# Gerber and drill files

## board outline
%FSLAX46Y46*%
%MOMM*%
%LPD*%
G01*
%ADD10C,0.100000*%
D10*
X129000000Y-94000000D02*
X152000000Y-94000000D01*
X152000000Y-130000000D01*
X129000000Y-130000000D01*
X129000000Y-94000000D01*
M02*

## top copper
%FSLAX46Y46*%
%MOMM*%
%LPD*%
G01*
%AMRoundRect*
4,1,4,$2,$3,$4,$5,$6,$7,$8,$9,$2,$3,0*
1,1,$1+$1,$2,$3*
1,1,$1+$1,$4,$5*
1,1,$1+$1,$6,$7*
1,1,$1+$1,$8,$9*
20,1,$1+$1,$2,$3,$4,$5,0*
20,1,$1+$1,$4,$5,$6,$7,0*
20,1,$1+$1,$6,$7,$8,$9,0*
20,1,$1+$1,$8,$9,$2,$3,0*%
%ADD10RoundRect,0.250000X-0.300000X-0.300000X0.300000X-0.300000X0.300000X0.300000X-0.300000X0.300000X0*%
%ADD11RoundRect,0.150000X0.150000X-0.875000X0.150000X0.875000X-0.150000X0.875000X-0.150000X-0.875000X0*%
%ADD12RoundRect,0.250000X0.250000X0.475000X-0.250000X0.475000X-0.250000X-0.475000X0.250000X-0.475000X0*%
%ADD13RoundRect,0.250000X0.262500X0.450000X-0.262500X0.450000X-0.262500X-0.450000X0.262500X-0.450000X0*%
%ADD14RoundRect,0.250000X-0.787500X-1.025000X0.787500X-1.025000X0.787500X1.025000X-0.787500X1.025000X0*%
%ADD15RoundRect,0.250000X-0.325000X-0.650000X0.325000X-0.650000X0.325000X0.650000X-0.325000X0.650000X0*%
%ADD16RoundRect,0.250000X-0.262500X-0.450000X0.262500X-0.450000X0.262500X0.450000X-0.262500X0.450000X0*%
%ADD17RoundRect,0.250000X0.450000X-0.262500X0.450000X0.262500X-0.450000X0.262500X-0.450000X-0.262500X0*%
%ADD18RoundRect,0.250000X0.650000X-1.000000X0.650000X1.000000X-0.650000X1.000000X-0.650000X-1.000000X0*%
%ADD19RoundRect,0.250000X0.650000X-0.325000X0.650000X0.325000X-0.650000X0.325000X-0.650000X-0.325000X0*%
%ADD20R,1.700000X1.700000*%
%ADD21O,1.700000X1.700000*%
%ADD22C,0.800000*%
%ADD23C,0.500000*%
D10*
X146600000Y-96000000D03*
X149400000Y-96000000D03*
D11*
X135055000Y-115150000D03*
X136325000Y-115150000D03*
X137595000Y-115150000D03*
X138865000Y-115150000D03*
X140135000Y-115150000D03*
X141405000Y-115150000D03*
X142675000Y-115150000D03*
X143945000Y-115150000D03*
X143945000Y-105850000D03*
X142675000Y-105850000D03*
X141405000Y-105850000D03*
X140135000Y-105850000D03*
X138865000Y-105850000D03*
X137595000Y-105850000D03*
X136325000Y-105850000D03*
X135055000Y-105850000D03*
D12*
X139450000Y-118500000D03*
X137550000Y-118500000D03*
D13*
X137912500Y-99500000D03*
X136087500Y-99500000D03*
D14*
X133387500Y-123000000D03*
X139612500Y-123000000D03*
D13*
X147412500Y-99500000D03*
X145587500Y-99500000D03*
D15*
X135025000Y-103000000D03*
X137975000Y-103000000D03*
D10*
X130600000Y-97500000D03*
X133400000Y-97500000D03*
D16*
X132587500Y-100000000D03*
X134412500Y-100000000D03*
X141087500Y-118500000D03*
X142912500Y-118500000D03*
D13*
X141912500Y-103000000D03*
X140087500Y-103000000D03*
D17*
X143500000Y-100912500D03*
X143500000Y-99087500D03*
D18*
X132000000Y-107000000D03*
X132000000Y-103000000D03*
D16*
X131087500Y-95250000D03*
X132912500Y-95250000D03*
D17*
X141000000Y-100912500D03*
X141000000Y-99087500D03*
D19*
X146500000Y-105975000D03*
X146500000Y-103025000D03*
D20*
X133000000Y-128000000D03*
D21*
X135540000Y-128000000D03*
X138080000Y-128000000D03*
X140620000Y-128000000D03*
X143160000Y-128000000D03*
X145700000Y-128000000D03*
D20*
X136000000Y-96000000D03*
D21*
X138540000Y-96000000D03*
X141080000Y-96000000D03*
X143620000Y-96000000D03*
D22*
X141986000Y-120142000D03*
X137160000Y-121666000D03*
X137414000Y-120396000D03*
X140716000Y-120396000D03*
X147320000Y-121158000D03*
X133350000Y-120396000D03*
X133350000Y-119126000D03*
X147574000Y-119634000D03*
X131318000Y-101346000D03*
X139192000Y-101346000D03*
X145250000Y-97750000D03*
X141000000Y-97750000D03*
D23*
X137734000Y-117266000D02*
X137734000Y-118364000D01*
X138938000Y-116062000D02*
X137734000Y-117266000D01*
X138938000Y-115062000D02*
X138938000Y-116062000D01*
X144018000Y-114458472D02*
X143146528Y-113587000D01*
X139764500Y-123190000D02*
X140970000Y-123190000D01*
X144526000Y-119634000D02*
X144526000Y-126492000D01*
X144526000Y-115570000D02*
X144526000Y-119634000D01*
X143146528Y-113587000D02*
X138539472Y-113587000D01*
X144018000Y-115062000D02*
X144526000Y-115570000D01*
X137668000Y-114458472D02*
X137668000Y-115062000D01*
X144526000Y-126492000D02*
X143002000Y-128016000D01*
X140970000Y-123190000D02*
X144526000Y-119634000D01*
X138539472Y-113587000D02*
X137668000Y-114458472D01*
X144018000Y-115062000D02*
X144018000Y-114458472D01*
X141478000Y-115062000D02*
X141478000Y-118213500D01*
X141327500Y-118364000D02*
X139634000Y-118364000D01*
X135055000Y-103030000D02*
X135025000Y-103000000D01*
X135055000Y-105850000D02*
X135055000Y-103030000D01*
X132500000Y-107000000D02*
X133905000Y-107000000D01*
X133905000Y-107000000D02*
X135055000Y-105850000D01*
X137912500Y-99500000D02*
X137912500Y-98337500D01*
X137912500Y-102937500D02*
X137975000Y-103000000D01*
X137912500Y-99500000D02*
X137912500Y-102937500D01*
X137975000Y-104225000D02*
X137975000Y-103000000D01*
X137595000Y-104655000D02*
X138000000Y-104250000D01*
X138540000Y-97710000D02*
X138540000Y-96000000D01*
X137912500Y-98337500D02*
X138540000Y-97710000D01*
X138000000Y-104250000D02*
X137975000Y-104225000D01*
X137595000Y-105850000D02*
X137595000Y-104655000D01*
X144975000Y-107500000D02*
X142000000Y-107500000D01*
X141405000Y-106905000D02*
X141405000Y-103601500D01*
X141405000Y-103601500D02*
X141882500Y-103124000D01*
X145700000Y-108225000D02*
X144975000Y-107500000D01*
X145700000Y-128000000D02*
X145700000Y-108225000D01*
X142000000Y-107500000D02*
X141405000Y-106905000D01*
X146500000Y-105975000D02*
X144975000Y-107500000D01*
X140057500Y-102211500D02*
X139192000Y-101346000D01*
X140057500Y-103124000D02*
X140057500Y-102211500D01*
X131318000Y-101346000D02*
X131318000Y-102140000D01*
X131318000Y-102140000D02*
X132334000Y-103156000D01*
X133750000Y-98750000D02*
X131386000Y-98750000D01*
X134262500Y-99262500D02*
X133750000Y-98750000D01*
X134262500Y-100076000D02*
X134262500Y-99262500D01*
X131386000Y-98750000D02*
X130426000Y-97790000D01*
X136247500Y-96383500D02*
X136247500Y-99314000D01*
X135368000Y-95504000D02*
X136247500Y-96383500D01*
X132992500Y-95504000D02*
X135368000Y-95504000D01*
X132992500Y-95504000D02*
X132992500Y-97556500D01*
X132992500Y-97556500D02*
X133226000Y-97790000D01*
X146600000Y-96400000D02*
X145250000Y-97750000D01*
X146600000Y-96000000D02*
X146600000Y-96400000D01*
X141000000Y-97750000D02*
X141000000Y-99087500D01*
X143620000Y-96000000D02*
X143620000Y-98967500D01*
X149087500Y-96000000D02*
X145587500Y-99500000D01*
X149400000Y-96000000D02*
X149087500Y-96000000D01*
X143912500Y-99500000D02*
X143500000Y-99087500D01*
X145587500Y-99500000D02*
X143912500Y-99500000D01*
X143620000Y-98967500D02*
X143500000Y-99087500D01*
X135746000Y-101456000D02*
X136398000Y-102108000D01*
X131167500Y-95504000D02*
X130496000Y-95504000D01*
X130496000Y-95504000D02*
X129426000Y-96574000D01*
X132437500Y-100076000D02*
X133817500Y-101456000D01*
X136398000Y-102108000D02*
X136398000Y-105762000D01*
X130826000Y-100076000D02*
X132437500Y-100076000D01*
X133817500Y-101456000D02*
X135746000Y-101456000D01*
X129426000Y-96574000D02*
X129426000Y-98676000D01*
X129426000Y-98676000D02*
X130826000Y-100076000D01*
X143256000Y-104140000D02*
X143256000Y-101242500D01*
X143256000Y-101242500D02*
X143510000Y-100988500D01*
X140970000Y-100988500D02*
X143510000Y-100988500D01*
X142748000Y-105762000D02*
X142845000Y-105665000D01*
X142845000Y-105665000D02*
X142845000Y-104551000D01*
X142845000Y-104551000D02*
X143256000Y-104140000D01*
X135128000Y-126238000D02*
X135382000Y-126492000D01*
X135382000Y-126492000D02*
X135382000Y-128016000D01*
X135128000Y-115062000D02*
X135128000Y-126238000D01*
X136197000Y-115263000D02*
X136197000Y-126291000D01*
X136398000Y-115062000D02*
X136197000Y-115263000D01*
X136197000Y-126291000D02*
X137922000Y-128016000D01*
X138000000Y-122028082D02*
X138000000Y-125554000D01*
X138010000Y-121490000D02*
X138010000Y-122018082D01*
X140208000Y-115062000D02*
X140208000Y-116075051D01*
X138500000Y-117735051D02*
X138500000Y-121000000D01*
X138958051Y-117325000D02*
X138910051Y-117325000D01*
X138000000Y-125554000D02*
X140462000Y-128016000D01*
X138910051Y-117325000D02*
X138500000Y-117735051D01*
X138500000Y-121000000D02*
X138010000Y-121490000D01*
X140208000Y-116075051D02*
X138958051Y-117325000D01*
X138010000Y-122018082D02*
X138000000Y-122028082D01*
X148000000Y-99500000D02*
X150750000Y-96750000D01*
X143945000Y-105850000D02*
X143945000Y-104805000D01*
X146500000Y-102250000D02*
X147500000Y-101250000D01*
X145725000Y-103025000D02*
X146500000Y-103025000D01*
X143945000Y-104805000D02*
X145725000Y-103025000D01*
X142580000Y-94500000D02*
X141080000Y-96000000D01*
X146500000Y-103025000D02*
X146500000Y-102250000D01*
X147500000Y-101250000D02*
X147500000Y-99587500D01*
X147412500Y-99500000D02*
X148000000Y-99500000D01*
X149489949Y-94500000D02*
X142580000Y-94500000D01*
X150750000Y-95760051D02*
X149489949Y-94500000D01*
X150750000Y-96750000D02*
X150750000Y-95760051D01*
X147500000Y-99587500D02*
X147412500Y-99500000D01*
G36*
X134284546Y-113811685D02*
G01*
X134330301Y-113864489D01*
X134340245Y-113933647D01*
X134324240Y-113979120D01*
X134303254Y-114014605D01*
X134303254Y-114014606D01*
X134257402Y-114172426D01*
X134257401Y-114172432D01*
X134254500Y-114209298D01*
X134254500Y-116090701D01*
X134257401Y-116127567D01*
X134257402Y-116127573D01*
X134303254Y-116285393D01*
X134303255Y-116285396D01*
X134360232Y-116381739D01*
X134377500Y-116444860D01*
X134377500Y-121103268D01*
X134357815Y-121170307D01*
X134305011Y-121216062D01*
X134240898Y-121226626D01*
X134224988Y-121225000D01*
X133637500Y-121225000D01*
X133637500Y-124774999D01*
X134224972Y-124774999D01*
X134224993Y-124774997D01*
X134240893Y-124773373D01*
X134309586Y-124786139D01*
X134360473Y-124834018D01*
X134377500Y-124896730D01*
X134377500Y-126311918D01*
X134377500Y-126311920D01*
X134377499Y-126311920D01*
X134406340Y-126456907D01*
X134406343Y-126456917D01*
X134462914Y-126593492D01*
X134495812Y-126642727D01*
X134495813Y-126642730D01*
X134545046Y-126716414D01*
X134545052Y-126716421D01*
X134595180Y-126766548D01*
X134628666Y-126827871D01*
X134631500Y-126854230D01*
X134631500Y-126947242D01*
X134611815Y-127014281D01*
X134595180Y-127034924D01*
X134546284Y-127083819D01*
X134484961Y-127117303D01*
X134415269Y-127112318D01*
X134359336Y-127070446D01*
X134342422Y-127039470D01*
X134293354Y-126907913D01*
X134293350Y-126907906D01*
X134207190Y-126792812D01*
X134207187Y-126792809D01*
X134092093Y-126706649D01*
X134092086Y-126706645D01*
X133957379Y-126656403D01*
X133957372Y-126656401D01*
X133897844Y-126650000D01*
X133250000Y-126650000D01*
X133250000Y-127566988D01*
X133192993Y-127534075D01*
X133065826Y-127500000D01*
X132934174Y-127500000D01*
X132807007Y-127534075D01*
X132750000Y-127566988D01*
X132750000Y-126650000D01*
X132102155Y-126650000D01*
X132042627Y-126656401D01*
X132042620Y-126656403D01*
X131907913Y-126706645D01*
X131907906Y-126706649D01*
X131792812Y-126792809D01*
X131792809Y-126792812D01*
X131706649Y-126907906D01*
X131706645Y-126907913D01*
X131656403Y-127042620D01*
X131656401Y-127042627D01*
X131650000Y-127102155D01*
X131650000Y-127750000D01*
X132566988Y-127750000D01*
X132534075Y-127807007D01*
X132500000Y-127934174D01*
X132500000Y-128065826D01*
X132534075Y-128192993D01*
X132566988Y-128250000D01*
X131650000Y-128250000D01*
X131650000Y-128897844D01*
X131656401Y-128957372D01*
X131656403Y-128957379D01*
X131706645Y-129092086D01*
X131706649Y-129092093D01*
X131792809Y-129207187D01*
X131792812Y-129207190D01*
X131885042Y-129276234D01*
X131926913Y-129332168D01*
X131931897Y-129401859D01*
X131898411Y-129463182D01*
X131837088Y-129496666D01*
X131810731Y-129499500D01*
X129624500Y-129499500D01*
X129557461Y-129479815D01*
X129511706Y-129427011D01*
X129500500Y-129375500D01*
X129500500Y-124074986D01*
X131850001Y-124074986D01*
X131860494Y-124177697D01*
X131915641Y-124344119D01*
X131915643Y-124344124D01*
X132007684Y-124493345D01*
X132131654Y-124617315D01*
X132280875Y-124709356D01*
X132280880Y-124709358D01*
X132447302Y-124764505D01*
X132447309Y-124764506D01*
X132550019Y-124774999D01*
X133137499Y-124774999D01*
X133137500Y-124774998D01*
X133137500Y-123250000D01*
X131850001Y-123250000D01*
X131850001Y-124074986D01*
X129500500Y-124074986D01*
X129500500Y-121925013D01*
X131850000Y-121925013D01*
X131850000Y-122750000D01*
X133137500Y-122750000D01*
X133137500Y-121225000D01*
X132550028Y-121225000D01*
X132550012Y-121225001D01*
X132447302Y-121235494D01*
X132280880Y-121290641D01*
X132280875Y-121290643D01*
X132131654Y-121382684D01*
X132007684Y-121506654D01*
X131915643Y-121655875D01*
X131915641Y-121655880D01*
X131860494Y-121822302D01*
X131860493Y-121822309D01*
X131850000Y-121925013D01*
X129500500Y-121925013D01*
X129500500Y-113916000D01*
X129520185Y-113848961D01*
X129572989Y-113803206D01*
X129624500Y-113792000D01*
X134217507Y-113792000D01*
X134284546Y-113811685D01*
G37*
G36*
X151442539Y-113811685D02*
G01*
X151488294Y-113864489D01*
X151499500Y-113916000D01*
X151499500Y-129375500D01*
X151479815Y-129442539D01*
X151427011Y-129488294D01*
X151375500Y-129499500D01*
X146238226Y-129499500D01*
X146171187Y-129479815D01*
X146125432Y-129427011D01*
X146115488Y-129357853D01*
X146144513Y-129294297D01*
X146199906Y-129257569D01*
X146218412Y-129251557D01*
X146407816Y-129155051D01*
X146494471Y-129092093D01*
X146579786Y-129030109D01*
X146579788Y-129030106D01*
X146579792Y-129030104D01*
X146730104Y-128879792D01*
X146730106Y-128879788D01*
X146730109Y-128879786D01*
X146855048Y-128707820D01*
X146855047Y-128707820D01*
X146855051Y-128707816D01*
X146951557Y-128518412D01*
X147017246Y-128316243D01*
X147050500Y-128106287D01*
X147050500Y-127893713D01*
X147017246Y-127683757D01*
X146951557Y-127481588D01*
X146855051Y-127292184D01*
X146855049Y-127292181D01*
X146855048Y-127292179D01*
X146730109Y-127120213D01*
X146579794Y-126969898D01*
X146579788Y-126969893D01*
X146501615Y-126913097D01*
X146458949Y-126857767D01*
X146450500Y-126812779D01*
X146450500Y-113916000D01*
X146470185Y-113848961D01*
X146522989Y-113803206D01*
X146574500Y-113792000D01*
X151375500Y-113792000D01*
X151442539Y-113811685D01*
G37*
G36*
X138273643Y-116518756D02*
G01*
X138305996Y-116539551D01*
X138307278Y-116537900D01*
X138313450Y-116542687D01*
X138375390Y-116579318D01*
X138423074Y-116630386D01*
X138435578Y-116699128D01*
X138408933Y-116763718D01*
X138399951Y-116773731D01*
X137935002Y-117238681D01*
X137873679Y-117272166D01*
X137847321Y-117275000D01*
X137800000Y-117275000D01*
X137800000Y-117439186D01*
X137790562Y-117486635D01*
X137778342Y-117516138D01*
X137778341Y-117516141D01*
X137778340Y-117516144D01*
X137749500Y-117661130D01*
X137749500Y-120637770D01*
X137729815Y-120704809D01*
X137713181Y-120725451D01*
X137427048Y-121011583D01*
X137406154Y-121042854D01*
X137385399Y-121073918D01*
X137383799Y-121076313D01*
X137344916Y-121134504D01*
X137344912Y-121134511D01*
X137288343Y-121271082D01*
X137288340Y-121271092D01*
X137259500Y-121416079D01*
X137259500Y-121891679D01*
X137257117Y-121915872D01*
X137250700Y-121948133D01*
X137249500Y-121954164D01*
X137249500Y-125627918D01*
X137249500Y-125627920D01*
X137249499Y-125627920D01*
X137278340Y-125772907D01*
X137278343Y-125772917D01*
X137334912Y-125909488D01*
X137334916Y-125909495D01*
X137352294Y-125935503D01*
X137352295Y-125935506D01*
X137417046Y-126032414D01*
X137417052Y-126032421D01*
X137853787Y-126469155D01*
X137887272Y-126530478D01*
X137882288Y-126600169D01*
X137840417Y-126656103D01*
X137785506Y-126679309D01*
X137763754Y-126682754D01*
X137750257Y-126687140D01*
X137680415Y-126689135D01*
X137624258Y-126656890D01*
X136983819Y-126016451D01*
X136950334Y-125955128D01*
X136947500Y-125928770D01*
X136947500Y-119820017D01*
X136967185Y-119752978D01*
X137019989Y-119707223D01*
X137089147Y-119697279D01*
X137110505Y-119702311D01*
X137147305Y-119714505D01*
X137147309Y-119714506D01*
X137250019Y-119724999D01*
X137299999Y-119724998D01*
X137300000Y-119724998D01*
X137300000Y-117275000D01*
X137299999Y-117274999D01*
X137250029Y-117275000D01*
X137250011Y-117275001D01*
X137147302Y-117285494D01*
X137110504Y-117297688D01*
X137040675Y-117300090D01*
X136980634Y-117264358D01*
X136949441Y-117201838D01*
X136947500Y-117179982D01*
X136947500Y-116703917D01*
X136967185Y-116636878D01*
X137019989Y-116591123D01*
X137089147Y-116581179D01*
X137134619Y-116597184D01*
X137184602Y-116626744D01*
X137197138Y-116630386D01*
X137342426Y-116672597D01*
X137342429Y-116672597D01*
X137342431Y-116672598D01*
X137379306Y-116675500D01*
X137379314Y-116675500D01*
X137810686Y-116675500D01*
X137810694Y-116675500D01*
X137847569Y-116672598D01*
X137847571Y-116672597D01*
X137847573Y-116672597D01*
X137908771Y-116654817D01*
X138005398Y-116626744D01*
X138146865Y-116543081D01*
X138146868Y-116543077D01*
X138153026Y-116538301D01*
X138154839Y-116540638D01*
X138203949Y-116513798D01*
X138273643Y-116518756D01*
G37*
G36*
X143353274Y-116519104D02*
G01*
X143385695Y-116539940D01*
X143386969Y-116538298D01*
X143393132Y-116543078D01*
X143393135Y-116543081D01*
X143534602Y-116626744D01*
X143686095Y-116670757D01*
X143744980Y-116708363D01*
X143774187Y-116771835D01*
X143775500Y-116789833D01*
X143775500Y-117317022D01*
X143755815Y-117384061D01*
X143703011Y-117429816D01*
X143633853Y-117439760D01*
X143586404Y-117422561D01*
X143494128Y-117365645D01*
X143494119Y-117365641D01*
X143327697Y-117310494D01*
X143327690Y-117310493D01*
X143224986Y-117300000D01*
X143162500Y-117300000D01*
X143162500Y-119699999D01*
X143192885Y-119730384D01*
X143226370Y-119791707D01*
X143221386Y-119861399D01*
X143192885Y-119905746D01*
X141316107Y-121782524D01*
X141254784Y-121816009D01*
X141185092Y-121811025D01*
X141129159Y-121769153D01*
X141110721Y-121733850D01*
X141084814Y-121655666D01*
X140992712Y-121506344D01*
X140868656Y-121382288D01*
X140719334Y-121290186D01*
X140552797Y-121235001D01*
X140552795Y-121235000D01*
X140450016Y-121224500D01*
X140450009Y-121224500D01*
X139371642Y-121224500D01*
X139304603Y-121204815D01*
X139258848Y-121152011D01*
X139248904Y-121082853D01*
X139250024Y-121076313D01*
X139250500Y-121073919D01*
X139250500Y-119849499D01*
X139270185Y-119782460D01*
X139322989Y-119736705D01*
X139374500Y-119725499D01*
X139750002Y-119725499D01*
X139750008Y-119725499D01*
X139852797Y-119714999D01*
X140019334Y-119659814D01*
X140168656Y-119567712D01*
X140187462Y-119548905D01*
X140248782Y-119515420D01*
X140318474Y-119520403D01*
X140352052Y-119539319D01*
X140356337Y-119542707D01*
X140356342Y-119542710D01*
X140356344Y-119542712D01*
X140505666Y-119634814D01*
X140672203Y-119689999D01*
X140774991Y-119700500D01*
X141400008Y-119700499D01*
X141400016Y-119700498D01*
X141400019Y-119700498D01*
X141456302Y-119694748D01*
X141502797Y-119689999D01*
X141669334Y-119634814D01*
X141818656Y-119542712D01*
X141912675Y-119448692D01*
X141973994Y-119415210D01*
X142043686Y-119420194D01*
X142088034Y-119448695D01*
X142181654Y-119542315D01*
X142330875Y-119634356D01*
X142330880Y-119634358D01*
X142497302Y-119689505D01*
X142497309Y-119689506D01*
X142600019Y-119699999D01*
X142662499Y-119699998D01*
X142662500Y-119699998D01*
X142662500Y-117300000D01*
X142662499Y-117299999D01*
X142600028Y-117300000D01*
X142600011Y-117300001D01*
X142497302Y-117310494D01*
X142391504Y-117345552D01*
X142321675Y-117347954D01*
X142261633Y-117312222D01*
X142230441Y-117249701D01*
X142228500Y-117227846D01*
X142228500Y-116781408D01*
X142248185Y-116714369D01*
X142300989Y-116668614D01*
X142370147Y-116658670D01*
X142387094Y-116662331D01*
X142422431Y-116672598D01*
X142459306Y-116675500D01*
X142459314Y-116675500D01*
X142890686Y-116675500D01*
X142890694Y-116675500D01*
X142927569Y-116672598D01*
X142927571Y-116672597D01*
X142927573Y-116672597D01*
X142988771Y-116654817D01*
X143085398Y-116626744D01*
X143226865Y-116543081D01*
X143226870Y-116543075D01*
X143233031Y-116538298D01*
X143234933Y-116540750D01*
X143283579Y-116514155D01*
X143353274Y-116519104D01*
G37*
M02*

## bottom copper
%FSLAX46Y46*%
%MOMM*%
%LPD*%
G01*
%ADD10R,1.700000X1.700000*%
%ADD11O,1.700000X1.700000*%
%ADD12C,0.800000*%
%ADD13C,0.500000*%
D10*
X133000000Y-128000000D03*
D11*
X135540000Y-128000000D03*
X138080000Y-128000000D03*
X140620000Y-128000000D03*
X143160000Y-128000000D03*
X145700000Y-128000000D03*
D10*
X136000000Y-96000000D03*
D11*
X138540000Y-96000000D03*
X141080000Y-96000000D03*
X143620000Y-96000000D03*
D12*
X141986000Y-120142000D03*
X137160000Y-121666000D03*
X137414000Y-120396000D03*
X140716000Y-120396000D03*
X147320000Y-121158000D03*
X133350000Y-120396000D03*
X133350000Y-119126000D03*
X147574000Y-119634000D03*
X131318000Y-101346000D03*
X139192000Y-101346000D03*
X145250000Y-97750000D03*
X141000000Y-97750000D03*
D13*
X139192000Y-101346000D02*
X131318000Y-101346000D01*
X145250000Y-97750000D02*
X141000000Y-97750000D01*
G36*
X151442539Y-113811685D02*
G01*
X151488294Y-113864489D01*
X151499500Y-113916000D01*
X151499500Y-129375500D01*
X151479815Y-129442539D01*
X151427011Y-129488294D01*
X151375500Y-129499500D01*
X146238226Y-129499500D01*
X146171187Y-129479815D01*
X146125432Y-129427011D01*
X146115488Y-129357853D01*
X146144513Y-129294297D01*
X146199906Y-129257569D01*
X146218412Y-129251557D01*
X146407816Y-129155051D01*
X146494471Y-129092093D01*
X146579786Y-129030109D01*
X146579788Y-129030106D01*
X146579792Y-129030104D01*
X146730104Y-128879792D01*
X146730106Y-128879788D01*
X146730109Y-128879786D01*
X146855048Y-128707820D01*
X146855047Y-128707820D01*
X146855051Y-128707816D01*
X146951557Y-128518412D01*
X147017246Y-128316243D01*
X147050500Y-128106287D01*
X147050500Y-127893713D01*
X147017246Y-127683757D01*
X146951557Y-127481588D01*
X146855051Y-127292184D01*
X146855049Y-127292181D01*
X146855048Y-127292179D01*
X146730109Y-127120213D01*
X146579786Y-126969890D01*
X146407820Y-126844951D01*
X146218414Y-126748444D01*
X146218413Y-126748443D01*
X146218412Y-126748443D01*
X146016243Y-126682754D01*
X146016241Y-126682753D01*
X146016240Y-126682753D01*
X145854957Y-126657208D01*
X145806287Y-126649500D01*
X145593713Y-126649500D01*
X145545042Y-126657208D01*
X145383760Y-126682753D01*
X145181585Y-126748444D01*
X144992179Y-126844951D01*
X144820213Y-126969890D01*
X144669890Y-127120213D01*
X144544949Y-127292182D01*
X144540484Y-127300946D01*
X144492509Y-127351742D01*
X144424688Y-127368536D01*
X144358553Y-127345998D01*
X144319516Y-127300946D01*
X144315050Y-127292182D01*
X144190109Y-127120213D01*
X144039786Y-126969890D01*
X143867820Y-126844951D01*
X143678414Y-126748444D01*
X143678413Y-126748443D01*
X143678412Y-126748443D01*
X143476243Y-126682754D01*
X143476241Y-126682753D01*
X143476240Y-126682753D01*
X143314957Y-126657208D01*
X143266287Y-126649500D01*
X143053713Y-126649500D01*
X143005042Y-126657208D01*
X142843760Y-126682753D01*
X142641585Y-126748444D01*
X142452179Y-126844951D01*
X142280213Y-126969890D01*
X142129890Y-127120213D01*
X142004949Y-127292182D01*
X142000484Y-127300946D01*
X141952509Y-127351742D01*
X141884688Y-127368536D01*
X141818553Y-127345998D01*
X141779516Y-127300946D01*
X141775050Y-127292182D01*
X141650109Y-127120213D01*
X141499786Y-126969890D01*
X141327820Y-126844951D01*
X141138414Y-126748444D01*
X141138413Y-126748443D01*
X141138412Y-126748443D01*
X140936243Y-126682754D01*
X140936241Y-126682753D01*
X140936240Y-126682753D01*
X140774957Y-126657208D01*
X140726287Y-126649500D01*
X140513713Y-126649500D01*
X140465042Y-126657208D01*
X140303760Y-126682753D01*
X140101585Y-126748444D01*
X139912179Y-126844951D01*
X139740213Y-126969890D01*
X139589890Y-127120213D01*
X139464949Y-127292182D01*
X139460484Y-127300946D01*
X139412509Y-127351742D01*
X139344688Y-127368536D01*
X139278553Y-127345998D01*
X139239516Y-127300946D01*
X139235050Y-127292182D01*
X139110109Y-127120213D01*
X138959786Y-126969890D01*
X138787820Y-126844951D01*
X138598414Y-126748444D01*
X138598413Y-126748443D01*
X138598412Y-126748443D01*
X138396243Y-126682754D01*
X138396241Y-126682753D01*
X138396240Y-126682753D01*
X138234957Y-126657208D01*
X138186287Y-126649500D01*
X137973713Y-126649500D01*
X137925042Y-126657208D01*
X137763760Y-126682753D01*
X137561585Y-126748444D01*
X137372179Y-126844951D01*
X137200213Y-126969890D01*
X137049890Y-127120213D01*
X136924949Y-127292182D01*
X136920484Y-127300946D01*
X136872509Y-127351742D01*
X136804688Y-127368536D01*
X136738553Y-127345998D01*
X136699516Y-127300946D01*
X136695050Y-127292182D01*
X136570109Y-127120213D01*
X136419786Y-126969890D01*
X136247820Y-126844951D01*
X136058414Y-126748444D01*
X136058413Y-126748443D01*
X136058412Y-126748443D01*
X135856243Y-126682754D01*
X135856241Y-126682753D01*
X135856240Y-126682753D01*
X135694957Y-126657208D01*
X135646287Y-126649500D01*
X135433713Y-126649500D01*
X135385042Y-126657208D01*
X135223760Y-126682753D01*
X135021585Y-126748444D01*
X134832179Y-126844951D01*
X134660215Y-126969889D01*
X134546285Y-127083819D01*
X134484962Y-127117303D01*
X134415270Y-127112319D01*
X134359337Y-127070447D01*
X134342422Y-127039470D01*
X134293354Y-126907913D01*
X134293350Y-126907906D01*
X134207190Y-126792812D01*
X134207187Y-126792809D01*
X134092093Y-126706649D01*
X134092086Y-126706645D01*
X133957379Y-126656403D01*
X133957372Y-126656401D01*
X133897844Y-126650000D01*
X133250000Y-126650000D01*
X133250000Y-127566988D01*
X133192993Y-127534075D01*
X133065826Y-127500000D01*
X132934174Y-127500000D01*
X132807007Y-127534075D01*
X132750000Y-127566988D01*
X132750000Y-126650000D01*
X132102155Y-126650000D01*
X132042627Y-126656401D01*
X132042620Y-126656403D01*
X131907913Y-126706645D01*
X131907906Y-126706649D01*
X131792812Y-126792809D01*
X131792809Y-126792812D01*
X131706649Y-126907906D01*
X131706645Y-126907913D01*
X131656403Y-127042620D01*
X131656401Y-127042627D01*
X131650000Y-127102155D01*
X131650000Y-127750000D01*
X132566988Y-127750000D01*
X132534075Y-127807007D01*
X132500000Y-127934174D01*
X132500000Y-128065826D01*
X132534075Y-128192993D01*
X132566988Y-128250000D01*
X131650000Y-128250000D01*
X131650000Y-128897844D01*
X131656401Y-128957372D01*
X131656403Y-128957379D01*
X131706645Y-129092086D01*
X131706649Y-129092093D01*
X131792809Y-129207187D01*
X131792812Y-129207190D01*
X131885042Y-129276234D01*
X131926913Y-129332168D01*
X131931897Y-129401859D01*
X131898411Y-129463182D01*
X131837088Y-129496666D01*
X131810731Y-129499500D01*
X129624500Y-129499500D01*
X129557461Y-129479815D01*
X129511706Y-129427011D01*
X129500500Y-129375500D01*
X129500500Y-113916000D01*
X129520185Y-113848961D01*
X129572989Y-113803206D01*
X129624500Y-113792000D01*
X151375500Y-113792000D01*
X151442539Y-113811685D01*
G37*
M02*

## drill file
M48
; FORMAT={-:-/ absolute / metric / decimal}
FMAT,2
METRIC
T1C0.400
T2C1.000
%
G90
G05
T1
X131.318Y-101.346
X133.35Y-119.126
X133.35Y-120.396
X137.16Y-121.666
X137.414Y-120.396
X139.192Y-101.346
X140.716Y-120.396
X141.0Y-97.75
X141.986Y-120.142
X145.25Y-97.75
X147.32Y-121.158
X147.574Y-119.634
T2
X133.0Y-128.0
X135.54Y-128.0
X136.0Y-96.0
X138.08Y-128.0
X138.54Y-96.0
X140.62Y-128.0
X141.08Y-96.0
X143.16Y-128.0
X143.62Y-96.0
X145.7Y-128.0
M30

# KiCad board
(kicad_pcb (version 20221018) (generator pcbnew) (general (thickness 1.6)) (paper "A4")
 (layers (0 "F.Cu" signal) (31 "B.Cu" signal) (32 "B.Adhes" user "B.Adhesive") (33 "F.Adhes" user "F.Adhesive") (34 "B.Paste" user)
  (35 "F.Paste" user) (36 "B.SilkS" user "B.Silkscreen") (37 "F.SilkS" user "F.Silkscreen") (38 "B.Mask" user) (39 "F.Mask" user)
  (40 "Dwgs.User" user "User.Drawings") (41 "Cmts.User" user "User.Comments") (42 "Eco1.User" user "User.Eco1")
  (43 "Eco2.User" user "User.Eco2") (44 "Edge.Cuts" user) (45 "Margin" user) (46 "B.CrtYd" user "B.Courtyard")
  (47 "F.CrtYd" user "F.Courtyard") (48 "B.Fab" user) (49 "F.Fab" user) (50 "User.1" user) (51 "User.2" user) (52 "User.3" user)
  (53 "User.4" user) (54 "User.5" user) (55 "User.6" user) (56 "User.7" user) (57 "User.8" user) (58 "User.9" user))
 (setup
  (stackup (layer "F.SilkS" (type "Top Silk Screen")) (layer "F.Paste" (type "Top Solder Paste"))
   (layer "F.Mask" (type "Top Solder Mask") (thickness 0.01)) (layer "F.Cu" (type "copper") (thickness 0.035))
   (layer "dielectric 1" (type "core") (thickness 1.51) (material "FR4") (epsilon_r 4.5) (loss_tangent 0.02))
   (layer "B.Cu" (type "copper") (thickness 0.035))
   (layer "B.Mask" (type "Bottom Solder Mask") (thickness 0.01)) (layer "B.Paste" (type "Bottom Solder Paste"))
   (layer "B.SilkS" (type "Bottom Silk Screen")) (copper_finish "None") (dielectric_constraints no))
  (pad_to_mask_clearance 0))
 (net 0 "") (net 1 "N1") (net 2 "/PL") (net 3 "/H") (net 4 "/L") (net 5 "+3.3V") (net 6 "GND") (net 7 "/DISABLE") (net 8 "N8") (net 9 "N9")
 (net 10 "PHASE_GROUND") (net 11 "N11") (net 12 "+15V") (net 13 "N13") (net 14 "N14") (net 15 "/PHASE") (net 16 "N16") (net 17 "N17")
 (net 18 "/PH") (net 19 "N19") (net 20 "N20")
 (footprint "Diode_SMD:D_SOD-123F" (layer "F.Cu") (at 148 96)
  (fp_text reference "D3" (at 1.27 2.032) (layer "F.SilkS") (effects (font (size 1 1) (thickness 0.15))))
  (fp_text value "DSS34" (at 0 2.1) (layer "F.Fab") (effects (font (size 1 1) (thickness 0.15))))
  (pad "1" smd roundrect (at -1.4 0) (size 1.1 1.1) (layers "F.Cu" "F.Paste" "F.Mask") (roundrect_rratio 0.2272727273) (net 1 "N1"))
  (pad "2" smd roundrect (at 1.4 0) (size 1.1 1.1) (layers "F.Cu" "F.Paste" "F.Mask") (roundrect_rratio 0.2272727273) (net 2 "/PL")))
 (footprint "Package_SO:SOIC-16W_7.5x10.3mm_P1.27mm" (layer "F.Cu") (at 139.5 110.5 90)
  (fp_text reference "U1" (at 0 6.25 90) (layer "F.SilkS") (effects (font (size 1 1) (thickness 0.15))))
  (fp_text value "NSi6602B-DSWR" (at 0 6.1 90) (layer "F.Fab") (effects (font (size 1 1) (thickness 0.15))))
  (pad "1" smd roundrect (at -4.65 -4.445 90) (size 2.05 0.6) (layers "F.Cu" "F.Paste" "F.Mask") (roundrect_rratio 0.25) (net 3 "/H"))
  (pad "2" smd roundrect (at -4.65 -3.175 90) (size 2.05 0.6) (layers "F.Cu" "F.Paste" "F.Mask") (roundrect_rratio 0.25) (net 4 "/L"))
  (pad "3" smd roundrect (at -4.65 -1.905 90) (size 2.05 0.6) (layers "F.Cu" "F.Paste" "F.Mask") (roundrect_rratio 0.25) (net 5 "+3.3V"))
  (pad "4" smd roundrect (at -4.65 -0.635 90) (size 2.05 0.6) (layers "F.Cu" "F.Paste" "F.Mask") (roundrect_rratio 0.25) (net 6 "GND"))
  (pad "5" smd roundrect (at -4.65 0.635 90) (size 2.05 0.6) (layers "F.Cu" "F.Paste" "F.Mask") (roundrect_rratio 0.25) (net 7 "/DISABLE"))
  (pad "6" smd roundrect (at -4.65 1.905 90) (size 2.05 0.6) (layers "F.Cu" "F.Paste" "F.Mask") (roundrect_rratio 0.25) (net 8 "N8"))
  (pad "7" smd roundrect (at -4.65 3.175 90) (size 2.05 0.6) (layers "F.Cu" "F.Paste" "F.Mask") (roundrect_rratio 0.25) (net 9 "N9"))
  (pad "8" smd roundrect (at -4.65 4.445 90) (size 2.05 0.6) (layers "F.Cu" "F.Paste" "F.Mask") (roundrect_rratio 0.25) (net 5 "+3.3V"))
  (pad "9" smd roundrect (at 4.65 4.445 90) (size 2.05 0.6) (layers "F.Cu" "F.Paste" "F.Mask") (roundrect_rratio 0.25)
   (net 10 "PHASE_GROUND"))
  (pad "10" smd roundrect (at 4.65 3.175 90) (size 2.05 0.6) (layers "F.Cu" "F.Paste" "F.Mask") (roundrect_rratio 0.25) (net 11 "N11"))
  (pad "11" smd roundrect (at 4.65 1.905 90) (size 2.05 0.6) (layers "F.Cu" "F.Paste" "F.Mask") (roundrect_rratio 0.25) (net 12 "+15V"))
  (pad "12" smd roundrect (at 4.65 0.635 90) (size 2.05 0.6) (layers "F.Cu" "F.Paste" "F.Mask") (roundrect_rratio 0.25) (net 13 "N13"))
  (pad "13" smd roundrect (at 4.65 -0.635 90) (size 2.05 0.6) (layers "F.Cu" "F.Paste" "F.Mask") (roundrect_rratio 0.25) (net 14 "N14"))
  (pad "14" smd roundrect (at 4.65 -1.905 90) (size 2.05 0.6) (layers "F.Cu" "F.Paste" "F.Mask") (roundrect_rratio 0.25) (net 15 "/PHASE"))
  (pad "15" smd roundrect (at 4.65 -3.175 90) (size 2.05 0.6) (layers "F.Cu" "F.Paste" "F.Mask") (roundrect_rratio 0.25) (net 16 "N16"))
  (pad "16" smd roundrect (at 4.65 -4.445 90) (size 2.05 0.6) (layers "F.Cu" "F.Paste" "F.Mask") (roundrect_rratio 0.25) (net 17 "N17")))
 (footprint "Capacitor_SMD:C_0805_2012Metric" (layer "F.Cu") (at 138.5 118.5 180)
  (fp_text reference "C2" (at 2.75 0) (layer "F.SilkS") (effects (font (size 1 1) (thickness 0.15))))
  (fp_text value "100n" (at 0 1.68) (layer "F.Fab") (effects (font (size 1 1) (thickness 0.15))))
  (pad "1" smd roundrect (at -0.95 0 180) (size 1 1.45) (layers "F.Cu" "F.Paste" "F.Mask") (roundrect_rratio 0.25) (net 8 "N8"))
  (pad "2" smd roundrect (at 0.95 0 180) (size 1 1.45) (layers "F.Cu" "F.Paste" "F.Mask") (roundrect_rratio 0.25) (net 6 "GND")))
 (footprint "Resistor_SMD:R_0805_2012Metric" (layer "F.Cu") (at 137 99.5 180)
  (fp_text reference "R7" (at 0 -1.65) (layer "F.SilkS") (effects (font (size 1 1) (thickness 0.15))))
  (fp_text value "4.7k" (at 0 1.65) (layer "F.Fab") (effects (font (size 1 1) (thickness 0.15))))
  (pad "1" smd roundrect (at -0.9125 0 180) (size 1.025 1.4) (layers "F.Cu" "F.Paste" "F.Mask") (roundrect_rratio 0.243902)
   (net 15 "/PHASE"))
  (pad "2" smd roundrect (at 0.9125 0 180) (size 1.025 1.4) (layers "F.Cu" "F.Paste" "F.Mask") (roundrect_rratio 0.243902) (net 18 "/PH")))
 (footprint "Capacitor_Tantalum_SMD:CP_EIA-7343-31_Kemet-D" (layer "F.Cu") (at 136.5 123)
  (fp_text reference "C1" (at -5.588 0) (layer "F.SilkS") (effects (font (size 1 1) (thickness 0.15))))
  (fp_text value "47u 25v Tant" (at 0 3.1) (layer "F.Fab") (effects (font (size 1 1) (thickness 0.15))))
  (pad "1" smd roundrect (at -3.1125 0) (size 2.075 2.55) (layers "F.Cu" "F.Paste" "F.Mask") (roundrect_rratio 0.120482) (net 6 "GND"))
  (pad "2" smd roundrect (at 3.1125 0) (size 2.075 2.55) (layers "F.Cu" "F.Paste" "F.Mask") (roundrect_rratio 0.120482) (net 5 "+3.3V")))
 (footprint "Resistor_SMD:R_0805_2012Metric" (layer "F.Cu") (at 146.5 99.5 180)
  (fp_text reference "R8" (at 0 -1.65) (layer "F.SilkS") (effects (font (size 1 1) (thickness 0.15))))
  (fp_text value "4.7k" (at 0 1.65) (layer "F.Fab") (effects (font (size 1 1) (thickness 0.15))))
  (pad "1" smd roundrect (at -0.9125 0 180) (size 1.025 1.4) (layers "F.Cu" "F.Paste" "F.Mask") (roundrect_rratio 0.243902)
   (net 10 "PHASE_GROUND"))
  (pad "2" smd roundrect (at 0.9125 0 180) (size 1.025 1.4) (layers "F.Cu" "F.Paste" "F.Mask") (roundrect_rratio 0.243902) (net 2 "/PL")))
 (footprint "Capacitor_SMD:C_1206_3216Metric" (layer "F.Cu") (at 136.5 103)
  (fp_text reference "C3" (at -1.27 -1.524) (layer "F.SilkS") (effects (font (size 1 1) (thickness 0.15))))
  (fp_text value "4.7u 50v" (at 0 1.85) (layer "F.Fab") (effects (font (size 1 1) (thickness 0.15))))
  (pad "1" smd roundrect (at -1.475 0) (size 1.15 1.8) (layers "F.Cu" "F.Paste" "F.Mask") (roundrect_rratio 0.217391) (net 17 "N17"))
  (pad "2" smd roundrect (at 1.475 0) (size 1.15 1.8) (layers "F.Cu" "F.Paste" "F.Mask") (roundrect_rratio 0.217391) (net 15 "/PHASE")))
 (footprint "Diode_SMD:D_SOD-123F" (layer "F.Cu") (at 132 97.5)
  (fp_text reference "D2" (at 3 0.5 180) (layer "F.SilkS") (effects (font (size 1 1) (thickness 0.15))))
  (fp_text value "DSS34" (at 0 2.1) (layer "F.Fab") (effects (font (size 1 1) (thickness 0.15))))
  (pad "1" smd roundrect (at -1.4 0) (size 1.1 1.1) (layers "F.Cu" "F.Paste" "F.Mask") (roundrect_rratio 0.2272727273) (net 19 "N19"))
  (pad "2" smd roundrect (at 1.4 0) (size 1.1 1.1) (layers "F.Cu" "F.Paste" "F.Mask") (roundrect_rratio 0.2272727273) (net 18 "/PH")))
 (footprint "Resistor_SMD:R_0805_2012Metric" (layer "F.Cu") (at 133.5 100)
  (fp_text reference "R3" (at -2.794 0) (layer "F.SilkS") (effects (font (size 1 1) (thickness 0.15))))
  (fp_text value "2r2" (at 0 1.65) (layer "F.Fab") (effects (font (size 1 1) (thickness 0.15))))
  (pad "1" smd roundrect (at -0.9125 0) (size 1.025 1.4) (layers "F.Cu" "F.Paste" "F.Mask") (roundrect_rratio 0.243902) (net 16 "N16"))
  (pad "2" smd roundrect (at 0.9125 0) (size 1.025 1.4) (layers "F.Cu" "F.Paste" "F.Mask") (roundrect_rratio 0.243902) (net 19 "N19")))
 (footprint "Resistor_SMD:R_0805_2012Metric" (layer "F.Cu") (at 142 118.5)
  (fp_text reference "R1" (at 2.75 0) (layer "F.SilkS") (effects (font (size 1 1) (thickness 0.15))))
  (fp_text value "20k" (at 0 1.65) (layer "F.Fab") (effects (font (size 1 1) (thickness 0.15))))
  (pad "1" smd roundrect (at -0.9125 0) (size 1.025 1.4) (layers "F.Cu" "F.Paste" "F.Mask") (roundrect_rratio 0.243902) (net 8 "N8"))
  (pad "2" smd roundrect (at 0.9125 0) (size 1.025 1.4) (layers "F.Cu" "F.Paste" "F.Mask") (roundrect_rratio 0.243902) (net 6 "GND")))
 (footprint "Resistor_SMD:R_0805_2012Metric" (layer "F.Cu") (at 141 103 180)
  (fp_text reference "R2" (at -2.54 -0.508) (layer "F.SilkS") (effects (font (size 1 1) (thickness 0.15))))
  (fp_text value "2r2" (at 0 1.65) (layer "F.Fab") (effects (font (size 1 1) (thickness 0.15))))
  (pad "1" smd roundrect (at -0.9125 0 180) (size 1.025 1.4) (layers "F.Cu" "F.Paste" "F.Mask") (roundrect_rratio 0.243902) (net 12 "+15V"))
  (pad "2" smd roundrect (at 0.9125 0 180) (size 1.025 1.4) (layers "F.Cu" "F.Paste" "F.Mask") (roundrect_rratio 0.243902) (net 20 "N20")))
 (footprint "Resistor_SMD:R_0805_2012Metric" (layer "F.Cu") (at 143.5 100 90)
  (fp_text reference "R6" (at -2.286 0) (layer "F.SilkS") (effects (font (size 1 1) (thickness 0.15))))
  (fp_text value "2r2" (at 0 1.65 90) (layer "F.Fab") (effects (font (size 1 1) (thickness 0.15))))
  (pad "1" smd roundrect (at -0.9125 0 90) (size 1.025 1.4) (layers "F.Cu" "F.Paste" "F.Mask") (roundrect_rratio 0.243902) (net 11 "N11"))
  (pad "2" smd roundrect (at 0.9125 0 90) (size 1.025 1.4) (layers "F.Cu" "F.Paste" "F.Mask") (roundrect_rratio 0.243902) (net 2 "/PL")))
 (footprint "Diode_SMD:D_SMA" (layer "F.Cu") (at 132 105 90)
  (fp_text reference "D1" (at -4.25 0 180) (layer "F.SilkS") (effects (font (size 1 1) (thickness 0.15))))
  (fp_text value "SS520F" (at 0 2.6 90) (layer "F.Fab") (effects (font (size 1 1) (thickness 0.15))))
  (pad "1" smd roundrect (at -2 0 90) (size 2.5 1.8) (layers "F.Cu" "F.Paste" "F.Mask") (roundrect_rratio 0.1388888889) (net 17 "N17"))
  (pad "2" smd roundrect (at 2 0 90) (size 2.5 1.8) (layers "F.Cu" "F.Paste" "F.Mask") (roundrect_rratio 0.1388888889) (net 20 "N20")))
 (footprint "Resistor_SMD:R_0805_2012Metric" (layer "F.Cu") (at 132 95.25)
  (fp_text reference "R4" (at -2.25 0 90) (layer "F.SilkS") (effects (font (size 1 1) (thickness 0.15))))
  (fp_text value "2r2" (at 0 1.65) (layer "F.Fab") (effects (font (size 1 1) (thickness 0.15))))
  (pad "1" smd roundrect (at -0.9125 0) (size 1.025 1.4) (layers "F.Cu" "F.Paste" "F.Mask") (roundrect_rratio 0.243902) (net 16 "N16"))
  (pad "2" smd roundrect (at 0.9125 0) (size 1.025 1.4) (layers "F.Cu" "F.Paste" "F.Mask") (roundrect_rratio 0.243902) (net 18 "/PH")))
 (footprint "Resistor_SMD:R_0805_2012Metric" (layer "F.Cu") (at 141 100 90)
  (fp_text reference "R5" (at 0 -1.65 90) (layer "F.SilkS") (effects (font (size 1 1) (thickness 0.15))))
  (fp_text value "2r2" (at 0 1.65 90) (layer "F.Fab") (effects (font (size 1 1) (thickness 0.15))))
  (pad "1" smd roundrect (at -0.9125 0 90) (size 1.025 1.4) (layers "F.Cu" "F.Paste" "F.Mask") (roundrect_rratio 0.243902) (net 11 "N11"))
  (pad "2" smd roundrect (at 0.9125 0 90) (size 1.025 1.4) (layers "F.Cu" "F.Paste" "F.Mask") (roundrect_rratio 0.243902) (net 1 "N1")))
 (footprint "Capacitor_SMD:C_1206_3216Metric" (layer "F.Cu") (at 146.5 104.5 90)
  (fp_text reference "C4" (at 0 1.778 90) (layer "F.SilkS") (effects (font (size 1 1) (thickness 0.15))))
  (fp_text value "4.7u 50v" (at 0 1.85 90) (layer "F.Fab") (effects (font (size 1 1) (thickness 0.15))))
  (pad "1" smd roundrect (at -1.475 0 90) (size 1.15 1.8) (layers "F.Cu" "F.Paste" "F.Mask") (roundrect_rratio 0.217391) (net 12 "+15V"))
  (pad "2" smd roundrect (at 1.475 0 90) (size 1.15 1.8) (layers "F.Cu" "F.Paste" "F.Mask") (roundrect_rratio 0.217391)
   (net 10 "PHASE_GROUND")))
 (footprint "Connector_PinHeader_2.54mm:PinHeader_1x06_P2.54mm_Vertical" (layer "B.Cu") (at 133 128 -90)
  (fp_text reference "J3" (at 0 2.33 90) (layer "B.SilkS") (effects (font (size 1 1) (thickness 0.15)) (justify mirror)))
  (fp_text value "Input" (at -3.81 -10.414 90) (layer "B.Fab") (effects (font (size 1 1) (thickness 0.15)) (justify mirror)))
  (pad "1" thru_hole rect (at 0 0 270) (size 1.7 1.7) (drill 1) (layers "*.Cu" "*.Mask") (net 6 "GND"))
  (pad "2" thru_hole oval (at 0 -2.54 270) (size 1.7 1.7) (drill 1) (layers "*.Cu" "*.Mask") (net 3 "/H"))
  (pad "3" thru_hole oval (at 0 -5.08 270) (size 1.7 1.7) (drill 1) (layers "*.Cu" "*.Mask") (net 4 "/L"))
  (pad "4" thru_hole oval (at 0 -7.62 270) (size 1.7 1.7) (drill 1) (layers "*.Cu" "*.Mask") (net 7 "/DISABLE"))
  (pad "5" thru_hole oval (at 0 -10.16 270) (size 1.7 1.7) (drill 1) (layers "*.Cu" "*.Mask") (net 5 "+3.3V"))
  (pad "6" thru_hole oval (at 0 -12.7 270) (size 1.7 1.7) (drill 1) (layers "*.Cu" "*.Mask") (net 12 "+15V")))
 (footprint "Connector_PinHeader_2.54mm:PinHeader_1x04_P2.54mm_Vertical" (layer "B.Cu") (at 136 96 -90)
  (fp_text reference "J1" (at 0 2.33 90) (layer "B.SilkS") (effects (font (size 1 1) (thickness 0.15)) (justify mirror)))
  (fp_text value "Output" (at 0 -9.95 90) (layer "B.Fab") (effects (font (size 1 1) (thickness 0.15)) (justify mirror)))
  (pad "1" thru_hole rect (at 0 0 270) (size 1.7 1.7) (drill 1) (layers "*.Cu" "*.Mask") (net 18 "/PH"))
  (pad "2" thru_hole oval (at 0 -2.54 270) (size 1.7 1.7) (drill 1) (layers "*.Cu" "*.Mask") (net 15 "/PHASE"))
  (pad "3" thru_hole oval (at 0 -5.08 270) (size 1.7 1.7) (drill 1) (layers "*.Cu" "*.Mask") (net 10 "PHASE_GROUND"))
  (pad "4" thru_hole oval (at 0 -7.62 270) (size 1.7 1.7) (drill 1) (layers "*.Cu" "*.Mask") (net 2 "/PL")))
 (gr_rect (start 129 94) (end 152 130) (stroke (width 0.1) (type default)) (fill none) (layer "Edge.Cuts"))
 (segment (start 137.734 117.266) (end 137.734 118.364) (width 0.5) (layer "F.Cu") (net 6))
 (segment (start 138.938 116.062) (end 137.734 117.266) (width 0.5) (layer "F.Cu") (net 6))
 (segment (start 138.938 115.062) (end 138.938 116.062) (width 0.5) (layer "F.Cu") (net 6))
 (via (at 141.986 120.142) (size 0.8) (drill 0.4) (layers "F.Cu" "B.Cu") (free) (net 6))
 (via (at 137.16 121.666) (size 0.8) (drill 0.4) (layers "F.Cu" "B.Cu") (free) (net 6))
 (via (at 137.414 120.396) (size 0.8) (drill 0.4) (layers "F.Cu" "B.Cu") (free) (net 6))
 (via (at 140.716 120.396) (size 0.8) (drill 0.4) (layers "F.Cu" "B.Cu") (free) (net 6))
 (via (at 147.32 121.158) (size 0.8) (drill 0.4) (layers "F.Cu" "B.Cu") (free) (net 6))
 (via (at 133.35 120.396) (size 0.8) (drill 0.4) (layers "F.Cu" "B.Cu") (free) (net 6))
 (via (at 133.35 119.126) (size 0.8) (drill 0.4) (layers "F.Cu" "B.Cu") (free) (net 6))
 (via (at 147.574 119.634) (size 0.8) (drill 0.4) (layers "F.Cu" "B.Cu") (free) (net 6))
 (segment (start 144.018 114.458472) (end 143.146528 113.587) (width 0.5) (layer "F.Cu") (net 5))
 (segment (start 139.7645 123.19) (end 140.97 123.19) (width 0.5) (layer "F.Cu") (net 5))
 (segment (start 144.526 119.634) (end 144.526 126.492) (width 0.5) (layer "F.Cu") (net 5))
 (segment (start 144.526 115.57) (end 144.526 119.634) (width 0.5) (layer "F.Cu") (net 5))
 (segment (start 143.146528 113.587) (end 138.539472 113.587) (width 0.5) (layer "F.Cu") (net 5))
 (segment (start 144.018 115.062) (end 144.526 115.57) (width 0.5) (layer "F.Cu") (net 5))
 (segment (start 137.668 114.458472) (end 137.668 115.062) (width 0.5) (layer "F.Cu") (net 5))
 (segment (start 144.526 126.492) (end 143.002 128.016) (width 0.5) (layer "F.Cu") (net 5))
 (segment (start 140.97 123.19) (end 144.526 119.634) (width 0.5) (layer "F.Cu") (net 5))
 (segment (start 138.539472 113.587) (end 137.668 114.458472) (width 0.5) (layer "F.Cu") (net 5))
 (segment (start 144.018 115.062) (end 144.018 114.458472) (width 0.5) (layer "F.Cu") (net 5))
 (segment (start 141.478 115.062) (end 141.478 118.2135) (width 0.5) (layer "F.Cu") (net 8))
 (segment (start 141.3275 118.364) (end 139.634 118.364) (width 0.5) (layer "F.Cu") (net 8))
 (segment (start 135.055 103.03) (end 135.025 103) (width 0.5) (layer "F.Cu") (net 17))
 (segment (start 135.055 105.85) (end 135.055 103.03) (width 0.5) (layer "F.Cu") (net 17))
 (segment (start 132.5 107) (end 133.905 107) (width 0.5) (layer "F.Cu") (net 17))
 (segment (start 133.905 107) (end 135.055 105.85) (width 0.5) (layer "F.Cu") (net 17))
 (segment (start 137.9125 99.5) (end 137.9125 98.3375) (width 0.5) (layer "F.Cu") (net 15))
 (segment (start 137.9125 102.9375) (end 137.975 103) (width 0.5) (layer "F.Cu") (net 15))
 (segment (start 137.9125 99.5) (end 137.9125 102.9375) (width 0.5) (layer "F.Cu") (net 15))
 (segment (start 137.975 104.225) (end 137.975 103) (width 0.5) (layer "F.Cu") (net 15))
 (segment (start 137.595 104.655) (end 138 104.25) (width 0.5) (layer "F.Cu") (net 15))
 (segment (start 138.54 97.71) (end 138.54 96) (width 0.5) (layer "F.Cu") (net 15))
 (segment (start 137.9125 98.3375) (end 138.54 97.71) (width 0.5) (layer "F.Cu") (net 15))
 (segment (start 138 104.25) (end 137.975 104.225) (width 0.5) (layer "F.Cu") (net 15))
 (segment (start 137.595 105.85) (end 137.595 104.655) (width 0.5) (layer "F.Cu") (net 15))
 (segment (start 144.975 107.5) (end 142 107.5) (width 0.5) (layer "F.Cu") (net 12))
 (segment (start 141.405 106.905) (end 141.405 103.6015) (width 0.5) (layer "F.Cu") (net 12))
 (segment (start 141.405 103.6015) (end 141.8825 103.124) (width 0.5) (layer "F.Cu") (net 12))
 (segment (start 145.7 108.225) (end 144.975 107.5) (width 0.5) (layer "F.Cu") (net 12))
 (segment (start 145.7 128) (end 145.7 108.225) (width 0.5) (layer "F.Cu") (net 12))
 (segment (start 142 107.5) (end 141.405 106.905) (width 0.5) (layer "F.Cu") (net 12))
 (segment (start 146.5 105.975) (end 144.975 107.5) (width 0.5) (layer "F.Cu") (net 12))
 (segment (start 140.0575 102.2115) (end 139.192 101.346) (width 0.5) (layer "F.Cu") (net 20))
 (segment (start 140.0575 103.124) (end 140.0575 102.2115) (width 0.5) (layer "F.Cu") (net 20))
 (segment (start 131.318 101.346) (end 131.318 102.14) (width 0.5) (layer "F.Cu") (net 20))
 (segment (start 131.318 102.14) (end 132.334 103.156) (width 0.5) (layer "F.Cu") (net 20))
 (via (at 131.318 101.346) (size 0.8) (drill 0.4) (layers "F.Cu" "B.Cu") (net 20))
 (via (at 139.192 101.346) (size 0.8) (drill 0.4) (layers "F.Cu" "B.Cu") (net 20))
 (segment (start 139.192 101.346) (end 131.318 101.346) (width 0.5) (layer "B.Cu") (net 20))
 (segment (start 133.75 98.75) (end 131.386 98.75) (width 0.5) (layer "F.Cu") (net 19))
 (segment (start 134.2625 99.2625) (end 133.75 98.75) (width 0.5) (layer "F.Cu") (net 19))
 (segment (start 134.2625 100.076) (end 134.2625 99.2625) (width 0.5) (layer "F.Cu") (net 19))
 (segment (start 131.386 98.75) (end 130.426 97.79) (width 0.5) (layer "F.Cu") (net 19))
 (segment (start 136.2475 96.3835) (end 136.2475 99.314) (width 0.5) (layer "F.Cu") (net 18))
 (segment (start 135.368 95.504) (end 136.2475 96.3835) (width 0.5) (layer "F.Cu") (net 18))
 (segment (start 132.9925 95.504) (end 135.368 95.504) (width 0.5) (layer "F.Cu") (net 18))
 (segment (start 132.9925 95.504) (end 132.9925 97.5565) (width 0.5) (layer "F.Cu") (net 18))
 (segment (start 132.9925 97.5565) (end 133.226 97.79) (width 0.5) (layer "F.Cu") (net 18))
 (segment (start 146.6 96.4) (end 145.25 97.75) (width 0.5) (layer "F.Cu") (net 1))
 (segment (start 146.6 96) (end 146.6 96.4) (width 0.5) (layer "F.Cu") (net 1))
 (segment (start 141 97.75) (end 141 99.0875) (width 0.5) (layer "F.Cu") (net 1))
 (via (at 145.25 97.75) (size 0.8) (drill 0.4) (layers "F.Cu" "B.Cu") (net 1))
 (via (at 141 97.75) (size 0.8) (drill 0.4) (layers "F.Cu" "B.Cu") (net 1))
 (segment (start 145.25 97.75) (end 141 97.75) (width 0.5) (layer "B.Cu") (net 1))
 (segment (start 143.62 96) (end 143.62 98.9675) (width 0.5) (layer "F.Cu") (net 2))
 (segment (start 149.0875 96) (end 145.5875 99.5) (width 0.5) (layer "F.Cu") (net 2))
 (segment (start 149.4 96) (end 149.0875 96) (width 0.5) (layer "F.Cu") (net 2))
 (segment (start 143.9125 99.5) (end 143.5 99.0875) (width 0.5) (layer "F.Cu") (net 2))
 (segment (start 145.5875 99.5) (end 143.9125 99.5) (width 0.5) (layer "F.Cu") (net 2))
 (segment (start 143.62 98.9675) (end 143.5 99.0875) (width 0.5) (layer "F.Cu") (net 2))
 (segment (start 135.746 101.456) (end 136.398 102.108) (width 0.5) (layer "F.Cu") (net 16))
 (segment (start 131.1675 95.504) (end 130.496 95.504) (width 0.5) (layer "F.Cu") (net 16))
 (segment (start 130.496 95.504) (end 129.426 96.574) (width 0.5) (layer "F.Cu") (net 16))
 (segment (start 132.4375 100.076) (end 133.8175 101.456) (width 0.5) (layer "F.Cu") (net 16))
 (segment (start 136.398 102.108) (end 136.398 105.762) (width 0.5) (layer "F.Cu") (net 16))
 (segment (start 130.826 100.076) (end 132.4375 100.076) (width 0.5) (layer "F.Cu") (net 16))
 (segment (start 133.8175 101.456) (end 135.746 101.456) (width 0.5) (layer "F.Cu") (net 16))
 (segment (start 129.426 96.574) (end 129.426 98.676) (width 0.5) (layer "F.Cu") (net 16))
 (segment (start 129.426 98.676) (end 130.826 100.076) (width 0.5) (layer "F.Cu") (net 16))
 (segment (start 143.256 104.14) (end 143.256 101.2425) (width 0.5) (layer "F.Cu") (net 11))
 (segment (start 143.256 101.2425) (end 143.51 100.9885) (width 0.5) (layer "F.Cu") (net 11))
 (segment (start 140.97 100.9885) (end 143.51 100.9885) (width 0.5) (layer "F.Cu") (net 11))
 (segment (start 142.748 105.762) (end 142.845 105.665) (width 0.5) (layer "F.Cu") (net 11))
 (segment (start 142.845 105.665) (end 142.845 104.551) (width 0.5) (layer "F.Cu") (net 11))
 (segment (start 142.845 104.551) (end 143.256 104.14) (width 0.5) (layer "F.Cu") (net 11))
 (segment (start 135.128 126.238) (end 135.382 126.492) (width 0.5) (layer "F.Cu") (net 3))
 (segment (start 135.382 126.492) (end 135.382 128.016) (width 0.5) (layer "F.Cu") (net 3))
 (segment (start 135.128 115.062) (end 135.128 126.238) (width 0.5) (layer "F.Cu") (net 3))
 (segment (start 136.197 115.263) (end 136.197 126.291) (width 0.5) (layer "F.Cu") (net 4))
 (segment (start 136.398 115.062) (end 136.197 115.263) (width 0.5) (layer "F.Cu") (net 4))
 (segment (start 136.197 126.291) (end 137.922 128.016) (width 0.5) (layer "F.Cu") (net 4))
 (segment (start 138 122.028082) (end 138 125.554) (width 0.5) (layer "F.Cu") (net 7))
 (segment (start 138.01 121.49) (end 138.01 122.018082) (width 0.5) (layer "F.Cu") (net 7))
 (segment (start 140.208 115.062) (end 140.208 116.075051) (width 0.5) (layer "F.Cu") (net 7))
 (segment (start 138.5 117.735051) (end 138.5 121) (width 0.5) (layer "F.Cu") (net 7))
 (segment (start 138.958051 117.325) (end 138.910051 117.325) (width 0.5) (layer "F.Cu") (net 7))
 (segment (start 138 125.554) (end 140.462 128.016) (width 0.5) (layer "F.Cu") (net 7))
 (segment (start 138.910051 117.325) (end 138.5 117.735051) (width 0.5) (layer "F.Cu") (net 7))
 (segment (start 138.5 121) (end 138.01 121.49) (width 0.5) (layer "F.Cu") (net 7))
 (segment (start 140.208 116.075051) (end 138.958051 117.325) (width 0.5) (layer "F.Cu") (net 7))
 (segment (start 138.01 122.018082) (end 138 122.028082) (width 0.5) (layer "F.Cu") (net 7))
 (segment (start 148 99.5) (end 150.75 96.75) (width 0.5) (layer "F.Cu") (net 10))
 (segment (start 143.945 105.85) (end 143.945 104.805) (width 0.5) (layer "F.Cu") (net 10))
 (segment (start 146.5 102.25) (end 147.5 101.25) (width 0.5) (layer "F.Cu") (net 10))
 (segment (start 145.725 103.025) (end 146.5 103.025) (width 0.5) (layer "F.Cu") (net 10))
 (segment (start 143.945 104.805) (end 145.725 103.025) (width 0.5) (layer "F.Cu") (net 10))
 (segment (start 142.58 94.5) (end 141.08 96) (width 0.5) (layer "F.Cu") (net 10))
 (segment (start 146.5 103.025) (end 146.5 102.25) (width 0.5) (layer "F.Cu") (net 10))
 (segment (start 147.5 101.25) (end 147.5 99.5875) (width 0.5) (layer "F.Cu") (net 10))
 (segment (start 147.4125 99.5) (end 148 99.5) (width 0.5) (layer "F.Cu") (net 10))
 (segment (start 149.489949 94.5) (end 142.58 94.5) (width 0.5) (layer "F.Cu") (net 10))
 (segment (start 150.75 95.760051) (end 149.489949 94.5) (width 0.5) (layer "F.Cu") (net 10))
 (segment (start 150.75 96.75) (end 150.75 95.760051) (width 0.5) (layer "F.Cu") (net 10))
 (segment (start 147.5 99.5875) (end 147.4125 99.5) (width 0.5) (layer "F.Cu") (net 10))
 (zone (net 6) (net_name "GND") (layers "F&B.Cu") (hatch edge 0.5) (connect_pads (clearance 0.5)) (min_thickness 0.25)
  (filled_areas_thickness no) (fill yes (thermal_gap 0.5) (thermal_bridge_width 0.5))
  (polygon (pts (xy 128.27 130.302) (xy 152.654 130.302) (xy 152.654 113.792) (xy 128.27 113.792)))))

